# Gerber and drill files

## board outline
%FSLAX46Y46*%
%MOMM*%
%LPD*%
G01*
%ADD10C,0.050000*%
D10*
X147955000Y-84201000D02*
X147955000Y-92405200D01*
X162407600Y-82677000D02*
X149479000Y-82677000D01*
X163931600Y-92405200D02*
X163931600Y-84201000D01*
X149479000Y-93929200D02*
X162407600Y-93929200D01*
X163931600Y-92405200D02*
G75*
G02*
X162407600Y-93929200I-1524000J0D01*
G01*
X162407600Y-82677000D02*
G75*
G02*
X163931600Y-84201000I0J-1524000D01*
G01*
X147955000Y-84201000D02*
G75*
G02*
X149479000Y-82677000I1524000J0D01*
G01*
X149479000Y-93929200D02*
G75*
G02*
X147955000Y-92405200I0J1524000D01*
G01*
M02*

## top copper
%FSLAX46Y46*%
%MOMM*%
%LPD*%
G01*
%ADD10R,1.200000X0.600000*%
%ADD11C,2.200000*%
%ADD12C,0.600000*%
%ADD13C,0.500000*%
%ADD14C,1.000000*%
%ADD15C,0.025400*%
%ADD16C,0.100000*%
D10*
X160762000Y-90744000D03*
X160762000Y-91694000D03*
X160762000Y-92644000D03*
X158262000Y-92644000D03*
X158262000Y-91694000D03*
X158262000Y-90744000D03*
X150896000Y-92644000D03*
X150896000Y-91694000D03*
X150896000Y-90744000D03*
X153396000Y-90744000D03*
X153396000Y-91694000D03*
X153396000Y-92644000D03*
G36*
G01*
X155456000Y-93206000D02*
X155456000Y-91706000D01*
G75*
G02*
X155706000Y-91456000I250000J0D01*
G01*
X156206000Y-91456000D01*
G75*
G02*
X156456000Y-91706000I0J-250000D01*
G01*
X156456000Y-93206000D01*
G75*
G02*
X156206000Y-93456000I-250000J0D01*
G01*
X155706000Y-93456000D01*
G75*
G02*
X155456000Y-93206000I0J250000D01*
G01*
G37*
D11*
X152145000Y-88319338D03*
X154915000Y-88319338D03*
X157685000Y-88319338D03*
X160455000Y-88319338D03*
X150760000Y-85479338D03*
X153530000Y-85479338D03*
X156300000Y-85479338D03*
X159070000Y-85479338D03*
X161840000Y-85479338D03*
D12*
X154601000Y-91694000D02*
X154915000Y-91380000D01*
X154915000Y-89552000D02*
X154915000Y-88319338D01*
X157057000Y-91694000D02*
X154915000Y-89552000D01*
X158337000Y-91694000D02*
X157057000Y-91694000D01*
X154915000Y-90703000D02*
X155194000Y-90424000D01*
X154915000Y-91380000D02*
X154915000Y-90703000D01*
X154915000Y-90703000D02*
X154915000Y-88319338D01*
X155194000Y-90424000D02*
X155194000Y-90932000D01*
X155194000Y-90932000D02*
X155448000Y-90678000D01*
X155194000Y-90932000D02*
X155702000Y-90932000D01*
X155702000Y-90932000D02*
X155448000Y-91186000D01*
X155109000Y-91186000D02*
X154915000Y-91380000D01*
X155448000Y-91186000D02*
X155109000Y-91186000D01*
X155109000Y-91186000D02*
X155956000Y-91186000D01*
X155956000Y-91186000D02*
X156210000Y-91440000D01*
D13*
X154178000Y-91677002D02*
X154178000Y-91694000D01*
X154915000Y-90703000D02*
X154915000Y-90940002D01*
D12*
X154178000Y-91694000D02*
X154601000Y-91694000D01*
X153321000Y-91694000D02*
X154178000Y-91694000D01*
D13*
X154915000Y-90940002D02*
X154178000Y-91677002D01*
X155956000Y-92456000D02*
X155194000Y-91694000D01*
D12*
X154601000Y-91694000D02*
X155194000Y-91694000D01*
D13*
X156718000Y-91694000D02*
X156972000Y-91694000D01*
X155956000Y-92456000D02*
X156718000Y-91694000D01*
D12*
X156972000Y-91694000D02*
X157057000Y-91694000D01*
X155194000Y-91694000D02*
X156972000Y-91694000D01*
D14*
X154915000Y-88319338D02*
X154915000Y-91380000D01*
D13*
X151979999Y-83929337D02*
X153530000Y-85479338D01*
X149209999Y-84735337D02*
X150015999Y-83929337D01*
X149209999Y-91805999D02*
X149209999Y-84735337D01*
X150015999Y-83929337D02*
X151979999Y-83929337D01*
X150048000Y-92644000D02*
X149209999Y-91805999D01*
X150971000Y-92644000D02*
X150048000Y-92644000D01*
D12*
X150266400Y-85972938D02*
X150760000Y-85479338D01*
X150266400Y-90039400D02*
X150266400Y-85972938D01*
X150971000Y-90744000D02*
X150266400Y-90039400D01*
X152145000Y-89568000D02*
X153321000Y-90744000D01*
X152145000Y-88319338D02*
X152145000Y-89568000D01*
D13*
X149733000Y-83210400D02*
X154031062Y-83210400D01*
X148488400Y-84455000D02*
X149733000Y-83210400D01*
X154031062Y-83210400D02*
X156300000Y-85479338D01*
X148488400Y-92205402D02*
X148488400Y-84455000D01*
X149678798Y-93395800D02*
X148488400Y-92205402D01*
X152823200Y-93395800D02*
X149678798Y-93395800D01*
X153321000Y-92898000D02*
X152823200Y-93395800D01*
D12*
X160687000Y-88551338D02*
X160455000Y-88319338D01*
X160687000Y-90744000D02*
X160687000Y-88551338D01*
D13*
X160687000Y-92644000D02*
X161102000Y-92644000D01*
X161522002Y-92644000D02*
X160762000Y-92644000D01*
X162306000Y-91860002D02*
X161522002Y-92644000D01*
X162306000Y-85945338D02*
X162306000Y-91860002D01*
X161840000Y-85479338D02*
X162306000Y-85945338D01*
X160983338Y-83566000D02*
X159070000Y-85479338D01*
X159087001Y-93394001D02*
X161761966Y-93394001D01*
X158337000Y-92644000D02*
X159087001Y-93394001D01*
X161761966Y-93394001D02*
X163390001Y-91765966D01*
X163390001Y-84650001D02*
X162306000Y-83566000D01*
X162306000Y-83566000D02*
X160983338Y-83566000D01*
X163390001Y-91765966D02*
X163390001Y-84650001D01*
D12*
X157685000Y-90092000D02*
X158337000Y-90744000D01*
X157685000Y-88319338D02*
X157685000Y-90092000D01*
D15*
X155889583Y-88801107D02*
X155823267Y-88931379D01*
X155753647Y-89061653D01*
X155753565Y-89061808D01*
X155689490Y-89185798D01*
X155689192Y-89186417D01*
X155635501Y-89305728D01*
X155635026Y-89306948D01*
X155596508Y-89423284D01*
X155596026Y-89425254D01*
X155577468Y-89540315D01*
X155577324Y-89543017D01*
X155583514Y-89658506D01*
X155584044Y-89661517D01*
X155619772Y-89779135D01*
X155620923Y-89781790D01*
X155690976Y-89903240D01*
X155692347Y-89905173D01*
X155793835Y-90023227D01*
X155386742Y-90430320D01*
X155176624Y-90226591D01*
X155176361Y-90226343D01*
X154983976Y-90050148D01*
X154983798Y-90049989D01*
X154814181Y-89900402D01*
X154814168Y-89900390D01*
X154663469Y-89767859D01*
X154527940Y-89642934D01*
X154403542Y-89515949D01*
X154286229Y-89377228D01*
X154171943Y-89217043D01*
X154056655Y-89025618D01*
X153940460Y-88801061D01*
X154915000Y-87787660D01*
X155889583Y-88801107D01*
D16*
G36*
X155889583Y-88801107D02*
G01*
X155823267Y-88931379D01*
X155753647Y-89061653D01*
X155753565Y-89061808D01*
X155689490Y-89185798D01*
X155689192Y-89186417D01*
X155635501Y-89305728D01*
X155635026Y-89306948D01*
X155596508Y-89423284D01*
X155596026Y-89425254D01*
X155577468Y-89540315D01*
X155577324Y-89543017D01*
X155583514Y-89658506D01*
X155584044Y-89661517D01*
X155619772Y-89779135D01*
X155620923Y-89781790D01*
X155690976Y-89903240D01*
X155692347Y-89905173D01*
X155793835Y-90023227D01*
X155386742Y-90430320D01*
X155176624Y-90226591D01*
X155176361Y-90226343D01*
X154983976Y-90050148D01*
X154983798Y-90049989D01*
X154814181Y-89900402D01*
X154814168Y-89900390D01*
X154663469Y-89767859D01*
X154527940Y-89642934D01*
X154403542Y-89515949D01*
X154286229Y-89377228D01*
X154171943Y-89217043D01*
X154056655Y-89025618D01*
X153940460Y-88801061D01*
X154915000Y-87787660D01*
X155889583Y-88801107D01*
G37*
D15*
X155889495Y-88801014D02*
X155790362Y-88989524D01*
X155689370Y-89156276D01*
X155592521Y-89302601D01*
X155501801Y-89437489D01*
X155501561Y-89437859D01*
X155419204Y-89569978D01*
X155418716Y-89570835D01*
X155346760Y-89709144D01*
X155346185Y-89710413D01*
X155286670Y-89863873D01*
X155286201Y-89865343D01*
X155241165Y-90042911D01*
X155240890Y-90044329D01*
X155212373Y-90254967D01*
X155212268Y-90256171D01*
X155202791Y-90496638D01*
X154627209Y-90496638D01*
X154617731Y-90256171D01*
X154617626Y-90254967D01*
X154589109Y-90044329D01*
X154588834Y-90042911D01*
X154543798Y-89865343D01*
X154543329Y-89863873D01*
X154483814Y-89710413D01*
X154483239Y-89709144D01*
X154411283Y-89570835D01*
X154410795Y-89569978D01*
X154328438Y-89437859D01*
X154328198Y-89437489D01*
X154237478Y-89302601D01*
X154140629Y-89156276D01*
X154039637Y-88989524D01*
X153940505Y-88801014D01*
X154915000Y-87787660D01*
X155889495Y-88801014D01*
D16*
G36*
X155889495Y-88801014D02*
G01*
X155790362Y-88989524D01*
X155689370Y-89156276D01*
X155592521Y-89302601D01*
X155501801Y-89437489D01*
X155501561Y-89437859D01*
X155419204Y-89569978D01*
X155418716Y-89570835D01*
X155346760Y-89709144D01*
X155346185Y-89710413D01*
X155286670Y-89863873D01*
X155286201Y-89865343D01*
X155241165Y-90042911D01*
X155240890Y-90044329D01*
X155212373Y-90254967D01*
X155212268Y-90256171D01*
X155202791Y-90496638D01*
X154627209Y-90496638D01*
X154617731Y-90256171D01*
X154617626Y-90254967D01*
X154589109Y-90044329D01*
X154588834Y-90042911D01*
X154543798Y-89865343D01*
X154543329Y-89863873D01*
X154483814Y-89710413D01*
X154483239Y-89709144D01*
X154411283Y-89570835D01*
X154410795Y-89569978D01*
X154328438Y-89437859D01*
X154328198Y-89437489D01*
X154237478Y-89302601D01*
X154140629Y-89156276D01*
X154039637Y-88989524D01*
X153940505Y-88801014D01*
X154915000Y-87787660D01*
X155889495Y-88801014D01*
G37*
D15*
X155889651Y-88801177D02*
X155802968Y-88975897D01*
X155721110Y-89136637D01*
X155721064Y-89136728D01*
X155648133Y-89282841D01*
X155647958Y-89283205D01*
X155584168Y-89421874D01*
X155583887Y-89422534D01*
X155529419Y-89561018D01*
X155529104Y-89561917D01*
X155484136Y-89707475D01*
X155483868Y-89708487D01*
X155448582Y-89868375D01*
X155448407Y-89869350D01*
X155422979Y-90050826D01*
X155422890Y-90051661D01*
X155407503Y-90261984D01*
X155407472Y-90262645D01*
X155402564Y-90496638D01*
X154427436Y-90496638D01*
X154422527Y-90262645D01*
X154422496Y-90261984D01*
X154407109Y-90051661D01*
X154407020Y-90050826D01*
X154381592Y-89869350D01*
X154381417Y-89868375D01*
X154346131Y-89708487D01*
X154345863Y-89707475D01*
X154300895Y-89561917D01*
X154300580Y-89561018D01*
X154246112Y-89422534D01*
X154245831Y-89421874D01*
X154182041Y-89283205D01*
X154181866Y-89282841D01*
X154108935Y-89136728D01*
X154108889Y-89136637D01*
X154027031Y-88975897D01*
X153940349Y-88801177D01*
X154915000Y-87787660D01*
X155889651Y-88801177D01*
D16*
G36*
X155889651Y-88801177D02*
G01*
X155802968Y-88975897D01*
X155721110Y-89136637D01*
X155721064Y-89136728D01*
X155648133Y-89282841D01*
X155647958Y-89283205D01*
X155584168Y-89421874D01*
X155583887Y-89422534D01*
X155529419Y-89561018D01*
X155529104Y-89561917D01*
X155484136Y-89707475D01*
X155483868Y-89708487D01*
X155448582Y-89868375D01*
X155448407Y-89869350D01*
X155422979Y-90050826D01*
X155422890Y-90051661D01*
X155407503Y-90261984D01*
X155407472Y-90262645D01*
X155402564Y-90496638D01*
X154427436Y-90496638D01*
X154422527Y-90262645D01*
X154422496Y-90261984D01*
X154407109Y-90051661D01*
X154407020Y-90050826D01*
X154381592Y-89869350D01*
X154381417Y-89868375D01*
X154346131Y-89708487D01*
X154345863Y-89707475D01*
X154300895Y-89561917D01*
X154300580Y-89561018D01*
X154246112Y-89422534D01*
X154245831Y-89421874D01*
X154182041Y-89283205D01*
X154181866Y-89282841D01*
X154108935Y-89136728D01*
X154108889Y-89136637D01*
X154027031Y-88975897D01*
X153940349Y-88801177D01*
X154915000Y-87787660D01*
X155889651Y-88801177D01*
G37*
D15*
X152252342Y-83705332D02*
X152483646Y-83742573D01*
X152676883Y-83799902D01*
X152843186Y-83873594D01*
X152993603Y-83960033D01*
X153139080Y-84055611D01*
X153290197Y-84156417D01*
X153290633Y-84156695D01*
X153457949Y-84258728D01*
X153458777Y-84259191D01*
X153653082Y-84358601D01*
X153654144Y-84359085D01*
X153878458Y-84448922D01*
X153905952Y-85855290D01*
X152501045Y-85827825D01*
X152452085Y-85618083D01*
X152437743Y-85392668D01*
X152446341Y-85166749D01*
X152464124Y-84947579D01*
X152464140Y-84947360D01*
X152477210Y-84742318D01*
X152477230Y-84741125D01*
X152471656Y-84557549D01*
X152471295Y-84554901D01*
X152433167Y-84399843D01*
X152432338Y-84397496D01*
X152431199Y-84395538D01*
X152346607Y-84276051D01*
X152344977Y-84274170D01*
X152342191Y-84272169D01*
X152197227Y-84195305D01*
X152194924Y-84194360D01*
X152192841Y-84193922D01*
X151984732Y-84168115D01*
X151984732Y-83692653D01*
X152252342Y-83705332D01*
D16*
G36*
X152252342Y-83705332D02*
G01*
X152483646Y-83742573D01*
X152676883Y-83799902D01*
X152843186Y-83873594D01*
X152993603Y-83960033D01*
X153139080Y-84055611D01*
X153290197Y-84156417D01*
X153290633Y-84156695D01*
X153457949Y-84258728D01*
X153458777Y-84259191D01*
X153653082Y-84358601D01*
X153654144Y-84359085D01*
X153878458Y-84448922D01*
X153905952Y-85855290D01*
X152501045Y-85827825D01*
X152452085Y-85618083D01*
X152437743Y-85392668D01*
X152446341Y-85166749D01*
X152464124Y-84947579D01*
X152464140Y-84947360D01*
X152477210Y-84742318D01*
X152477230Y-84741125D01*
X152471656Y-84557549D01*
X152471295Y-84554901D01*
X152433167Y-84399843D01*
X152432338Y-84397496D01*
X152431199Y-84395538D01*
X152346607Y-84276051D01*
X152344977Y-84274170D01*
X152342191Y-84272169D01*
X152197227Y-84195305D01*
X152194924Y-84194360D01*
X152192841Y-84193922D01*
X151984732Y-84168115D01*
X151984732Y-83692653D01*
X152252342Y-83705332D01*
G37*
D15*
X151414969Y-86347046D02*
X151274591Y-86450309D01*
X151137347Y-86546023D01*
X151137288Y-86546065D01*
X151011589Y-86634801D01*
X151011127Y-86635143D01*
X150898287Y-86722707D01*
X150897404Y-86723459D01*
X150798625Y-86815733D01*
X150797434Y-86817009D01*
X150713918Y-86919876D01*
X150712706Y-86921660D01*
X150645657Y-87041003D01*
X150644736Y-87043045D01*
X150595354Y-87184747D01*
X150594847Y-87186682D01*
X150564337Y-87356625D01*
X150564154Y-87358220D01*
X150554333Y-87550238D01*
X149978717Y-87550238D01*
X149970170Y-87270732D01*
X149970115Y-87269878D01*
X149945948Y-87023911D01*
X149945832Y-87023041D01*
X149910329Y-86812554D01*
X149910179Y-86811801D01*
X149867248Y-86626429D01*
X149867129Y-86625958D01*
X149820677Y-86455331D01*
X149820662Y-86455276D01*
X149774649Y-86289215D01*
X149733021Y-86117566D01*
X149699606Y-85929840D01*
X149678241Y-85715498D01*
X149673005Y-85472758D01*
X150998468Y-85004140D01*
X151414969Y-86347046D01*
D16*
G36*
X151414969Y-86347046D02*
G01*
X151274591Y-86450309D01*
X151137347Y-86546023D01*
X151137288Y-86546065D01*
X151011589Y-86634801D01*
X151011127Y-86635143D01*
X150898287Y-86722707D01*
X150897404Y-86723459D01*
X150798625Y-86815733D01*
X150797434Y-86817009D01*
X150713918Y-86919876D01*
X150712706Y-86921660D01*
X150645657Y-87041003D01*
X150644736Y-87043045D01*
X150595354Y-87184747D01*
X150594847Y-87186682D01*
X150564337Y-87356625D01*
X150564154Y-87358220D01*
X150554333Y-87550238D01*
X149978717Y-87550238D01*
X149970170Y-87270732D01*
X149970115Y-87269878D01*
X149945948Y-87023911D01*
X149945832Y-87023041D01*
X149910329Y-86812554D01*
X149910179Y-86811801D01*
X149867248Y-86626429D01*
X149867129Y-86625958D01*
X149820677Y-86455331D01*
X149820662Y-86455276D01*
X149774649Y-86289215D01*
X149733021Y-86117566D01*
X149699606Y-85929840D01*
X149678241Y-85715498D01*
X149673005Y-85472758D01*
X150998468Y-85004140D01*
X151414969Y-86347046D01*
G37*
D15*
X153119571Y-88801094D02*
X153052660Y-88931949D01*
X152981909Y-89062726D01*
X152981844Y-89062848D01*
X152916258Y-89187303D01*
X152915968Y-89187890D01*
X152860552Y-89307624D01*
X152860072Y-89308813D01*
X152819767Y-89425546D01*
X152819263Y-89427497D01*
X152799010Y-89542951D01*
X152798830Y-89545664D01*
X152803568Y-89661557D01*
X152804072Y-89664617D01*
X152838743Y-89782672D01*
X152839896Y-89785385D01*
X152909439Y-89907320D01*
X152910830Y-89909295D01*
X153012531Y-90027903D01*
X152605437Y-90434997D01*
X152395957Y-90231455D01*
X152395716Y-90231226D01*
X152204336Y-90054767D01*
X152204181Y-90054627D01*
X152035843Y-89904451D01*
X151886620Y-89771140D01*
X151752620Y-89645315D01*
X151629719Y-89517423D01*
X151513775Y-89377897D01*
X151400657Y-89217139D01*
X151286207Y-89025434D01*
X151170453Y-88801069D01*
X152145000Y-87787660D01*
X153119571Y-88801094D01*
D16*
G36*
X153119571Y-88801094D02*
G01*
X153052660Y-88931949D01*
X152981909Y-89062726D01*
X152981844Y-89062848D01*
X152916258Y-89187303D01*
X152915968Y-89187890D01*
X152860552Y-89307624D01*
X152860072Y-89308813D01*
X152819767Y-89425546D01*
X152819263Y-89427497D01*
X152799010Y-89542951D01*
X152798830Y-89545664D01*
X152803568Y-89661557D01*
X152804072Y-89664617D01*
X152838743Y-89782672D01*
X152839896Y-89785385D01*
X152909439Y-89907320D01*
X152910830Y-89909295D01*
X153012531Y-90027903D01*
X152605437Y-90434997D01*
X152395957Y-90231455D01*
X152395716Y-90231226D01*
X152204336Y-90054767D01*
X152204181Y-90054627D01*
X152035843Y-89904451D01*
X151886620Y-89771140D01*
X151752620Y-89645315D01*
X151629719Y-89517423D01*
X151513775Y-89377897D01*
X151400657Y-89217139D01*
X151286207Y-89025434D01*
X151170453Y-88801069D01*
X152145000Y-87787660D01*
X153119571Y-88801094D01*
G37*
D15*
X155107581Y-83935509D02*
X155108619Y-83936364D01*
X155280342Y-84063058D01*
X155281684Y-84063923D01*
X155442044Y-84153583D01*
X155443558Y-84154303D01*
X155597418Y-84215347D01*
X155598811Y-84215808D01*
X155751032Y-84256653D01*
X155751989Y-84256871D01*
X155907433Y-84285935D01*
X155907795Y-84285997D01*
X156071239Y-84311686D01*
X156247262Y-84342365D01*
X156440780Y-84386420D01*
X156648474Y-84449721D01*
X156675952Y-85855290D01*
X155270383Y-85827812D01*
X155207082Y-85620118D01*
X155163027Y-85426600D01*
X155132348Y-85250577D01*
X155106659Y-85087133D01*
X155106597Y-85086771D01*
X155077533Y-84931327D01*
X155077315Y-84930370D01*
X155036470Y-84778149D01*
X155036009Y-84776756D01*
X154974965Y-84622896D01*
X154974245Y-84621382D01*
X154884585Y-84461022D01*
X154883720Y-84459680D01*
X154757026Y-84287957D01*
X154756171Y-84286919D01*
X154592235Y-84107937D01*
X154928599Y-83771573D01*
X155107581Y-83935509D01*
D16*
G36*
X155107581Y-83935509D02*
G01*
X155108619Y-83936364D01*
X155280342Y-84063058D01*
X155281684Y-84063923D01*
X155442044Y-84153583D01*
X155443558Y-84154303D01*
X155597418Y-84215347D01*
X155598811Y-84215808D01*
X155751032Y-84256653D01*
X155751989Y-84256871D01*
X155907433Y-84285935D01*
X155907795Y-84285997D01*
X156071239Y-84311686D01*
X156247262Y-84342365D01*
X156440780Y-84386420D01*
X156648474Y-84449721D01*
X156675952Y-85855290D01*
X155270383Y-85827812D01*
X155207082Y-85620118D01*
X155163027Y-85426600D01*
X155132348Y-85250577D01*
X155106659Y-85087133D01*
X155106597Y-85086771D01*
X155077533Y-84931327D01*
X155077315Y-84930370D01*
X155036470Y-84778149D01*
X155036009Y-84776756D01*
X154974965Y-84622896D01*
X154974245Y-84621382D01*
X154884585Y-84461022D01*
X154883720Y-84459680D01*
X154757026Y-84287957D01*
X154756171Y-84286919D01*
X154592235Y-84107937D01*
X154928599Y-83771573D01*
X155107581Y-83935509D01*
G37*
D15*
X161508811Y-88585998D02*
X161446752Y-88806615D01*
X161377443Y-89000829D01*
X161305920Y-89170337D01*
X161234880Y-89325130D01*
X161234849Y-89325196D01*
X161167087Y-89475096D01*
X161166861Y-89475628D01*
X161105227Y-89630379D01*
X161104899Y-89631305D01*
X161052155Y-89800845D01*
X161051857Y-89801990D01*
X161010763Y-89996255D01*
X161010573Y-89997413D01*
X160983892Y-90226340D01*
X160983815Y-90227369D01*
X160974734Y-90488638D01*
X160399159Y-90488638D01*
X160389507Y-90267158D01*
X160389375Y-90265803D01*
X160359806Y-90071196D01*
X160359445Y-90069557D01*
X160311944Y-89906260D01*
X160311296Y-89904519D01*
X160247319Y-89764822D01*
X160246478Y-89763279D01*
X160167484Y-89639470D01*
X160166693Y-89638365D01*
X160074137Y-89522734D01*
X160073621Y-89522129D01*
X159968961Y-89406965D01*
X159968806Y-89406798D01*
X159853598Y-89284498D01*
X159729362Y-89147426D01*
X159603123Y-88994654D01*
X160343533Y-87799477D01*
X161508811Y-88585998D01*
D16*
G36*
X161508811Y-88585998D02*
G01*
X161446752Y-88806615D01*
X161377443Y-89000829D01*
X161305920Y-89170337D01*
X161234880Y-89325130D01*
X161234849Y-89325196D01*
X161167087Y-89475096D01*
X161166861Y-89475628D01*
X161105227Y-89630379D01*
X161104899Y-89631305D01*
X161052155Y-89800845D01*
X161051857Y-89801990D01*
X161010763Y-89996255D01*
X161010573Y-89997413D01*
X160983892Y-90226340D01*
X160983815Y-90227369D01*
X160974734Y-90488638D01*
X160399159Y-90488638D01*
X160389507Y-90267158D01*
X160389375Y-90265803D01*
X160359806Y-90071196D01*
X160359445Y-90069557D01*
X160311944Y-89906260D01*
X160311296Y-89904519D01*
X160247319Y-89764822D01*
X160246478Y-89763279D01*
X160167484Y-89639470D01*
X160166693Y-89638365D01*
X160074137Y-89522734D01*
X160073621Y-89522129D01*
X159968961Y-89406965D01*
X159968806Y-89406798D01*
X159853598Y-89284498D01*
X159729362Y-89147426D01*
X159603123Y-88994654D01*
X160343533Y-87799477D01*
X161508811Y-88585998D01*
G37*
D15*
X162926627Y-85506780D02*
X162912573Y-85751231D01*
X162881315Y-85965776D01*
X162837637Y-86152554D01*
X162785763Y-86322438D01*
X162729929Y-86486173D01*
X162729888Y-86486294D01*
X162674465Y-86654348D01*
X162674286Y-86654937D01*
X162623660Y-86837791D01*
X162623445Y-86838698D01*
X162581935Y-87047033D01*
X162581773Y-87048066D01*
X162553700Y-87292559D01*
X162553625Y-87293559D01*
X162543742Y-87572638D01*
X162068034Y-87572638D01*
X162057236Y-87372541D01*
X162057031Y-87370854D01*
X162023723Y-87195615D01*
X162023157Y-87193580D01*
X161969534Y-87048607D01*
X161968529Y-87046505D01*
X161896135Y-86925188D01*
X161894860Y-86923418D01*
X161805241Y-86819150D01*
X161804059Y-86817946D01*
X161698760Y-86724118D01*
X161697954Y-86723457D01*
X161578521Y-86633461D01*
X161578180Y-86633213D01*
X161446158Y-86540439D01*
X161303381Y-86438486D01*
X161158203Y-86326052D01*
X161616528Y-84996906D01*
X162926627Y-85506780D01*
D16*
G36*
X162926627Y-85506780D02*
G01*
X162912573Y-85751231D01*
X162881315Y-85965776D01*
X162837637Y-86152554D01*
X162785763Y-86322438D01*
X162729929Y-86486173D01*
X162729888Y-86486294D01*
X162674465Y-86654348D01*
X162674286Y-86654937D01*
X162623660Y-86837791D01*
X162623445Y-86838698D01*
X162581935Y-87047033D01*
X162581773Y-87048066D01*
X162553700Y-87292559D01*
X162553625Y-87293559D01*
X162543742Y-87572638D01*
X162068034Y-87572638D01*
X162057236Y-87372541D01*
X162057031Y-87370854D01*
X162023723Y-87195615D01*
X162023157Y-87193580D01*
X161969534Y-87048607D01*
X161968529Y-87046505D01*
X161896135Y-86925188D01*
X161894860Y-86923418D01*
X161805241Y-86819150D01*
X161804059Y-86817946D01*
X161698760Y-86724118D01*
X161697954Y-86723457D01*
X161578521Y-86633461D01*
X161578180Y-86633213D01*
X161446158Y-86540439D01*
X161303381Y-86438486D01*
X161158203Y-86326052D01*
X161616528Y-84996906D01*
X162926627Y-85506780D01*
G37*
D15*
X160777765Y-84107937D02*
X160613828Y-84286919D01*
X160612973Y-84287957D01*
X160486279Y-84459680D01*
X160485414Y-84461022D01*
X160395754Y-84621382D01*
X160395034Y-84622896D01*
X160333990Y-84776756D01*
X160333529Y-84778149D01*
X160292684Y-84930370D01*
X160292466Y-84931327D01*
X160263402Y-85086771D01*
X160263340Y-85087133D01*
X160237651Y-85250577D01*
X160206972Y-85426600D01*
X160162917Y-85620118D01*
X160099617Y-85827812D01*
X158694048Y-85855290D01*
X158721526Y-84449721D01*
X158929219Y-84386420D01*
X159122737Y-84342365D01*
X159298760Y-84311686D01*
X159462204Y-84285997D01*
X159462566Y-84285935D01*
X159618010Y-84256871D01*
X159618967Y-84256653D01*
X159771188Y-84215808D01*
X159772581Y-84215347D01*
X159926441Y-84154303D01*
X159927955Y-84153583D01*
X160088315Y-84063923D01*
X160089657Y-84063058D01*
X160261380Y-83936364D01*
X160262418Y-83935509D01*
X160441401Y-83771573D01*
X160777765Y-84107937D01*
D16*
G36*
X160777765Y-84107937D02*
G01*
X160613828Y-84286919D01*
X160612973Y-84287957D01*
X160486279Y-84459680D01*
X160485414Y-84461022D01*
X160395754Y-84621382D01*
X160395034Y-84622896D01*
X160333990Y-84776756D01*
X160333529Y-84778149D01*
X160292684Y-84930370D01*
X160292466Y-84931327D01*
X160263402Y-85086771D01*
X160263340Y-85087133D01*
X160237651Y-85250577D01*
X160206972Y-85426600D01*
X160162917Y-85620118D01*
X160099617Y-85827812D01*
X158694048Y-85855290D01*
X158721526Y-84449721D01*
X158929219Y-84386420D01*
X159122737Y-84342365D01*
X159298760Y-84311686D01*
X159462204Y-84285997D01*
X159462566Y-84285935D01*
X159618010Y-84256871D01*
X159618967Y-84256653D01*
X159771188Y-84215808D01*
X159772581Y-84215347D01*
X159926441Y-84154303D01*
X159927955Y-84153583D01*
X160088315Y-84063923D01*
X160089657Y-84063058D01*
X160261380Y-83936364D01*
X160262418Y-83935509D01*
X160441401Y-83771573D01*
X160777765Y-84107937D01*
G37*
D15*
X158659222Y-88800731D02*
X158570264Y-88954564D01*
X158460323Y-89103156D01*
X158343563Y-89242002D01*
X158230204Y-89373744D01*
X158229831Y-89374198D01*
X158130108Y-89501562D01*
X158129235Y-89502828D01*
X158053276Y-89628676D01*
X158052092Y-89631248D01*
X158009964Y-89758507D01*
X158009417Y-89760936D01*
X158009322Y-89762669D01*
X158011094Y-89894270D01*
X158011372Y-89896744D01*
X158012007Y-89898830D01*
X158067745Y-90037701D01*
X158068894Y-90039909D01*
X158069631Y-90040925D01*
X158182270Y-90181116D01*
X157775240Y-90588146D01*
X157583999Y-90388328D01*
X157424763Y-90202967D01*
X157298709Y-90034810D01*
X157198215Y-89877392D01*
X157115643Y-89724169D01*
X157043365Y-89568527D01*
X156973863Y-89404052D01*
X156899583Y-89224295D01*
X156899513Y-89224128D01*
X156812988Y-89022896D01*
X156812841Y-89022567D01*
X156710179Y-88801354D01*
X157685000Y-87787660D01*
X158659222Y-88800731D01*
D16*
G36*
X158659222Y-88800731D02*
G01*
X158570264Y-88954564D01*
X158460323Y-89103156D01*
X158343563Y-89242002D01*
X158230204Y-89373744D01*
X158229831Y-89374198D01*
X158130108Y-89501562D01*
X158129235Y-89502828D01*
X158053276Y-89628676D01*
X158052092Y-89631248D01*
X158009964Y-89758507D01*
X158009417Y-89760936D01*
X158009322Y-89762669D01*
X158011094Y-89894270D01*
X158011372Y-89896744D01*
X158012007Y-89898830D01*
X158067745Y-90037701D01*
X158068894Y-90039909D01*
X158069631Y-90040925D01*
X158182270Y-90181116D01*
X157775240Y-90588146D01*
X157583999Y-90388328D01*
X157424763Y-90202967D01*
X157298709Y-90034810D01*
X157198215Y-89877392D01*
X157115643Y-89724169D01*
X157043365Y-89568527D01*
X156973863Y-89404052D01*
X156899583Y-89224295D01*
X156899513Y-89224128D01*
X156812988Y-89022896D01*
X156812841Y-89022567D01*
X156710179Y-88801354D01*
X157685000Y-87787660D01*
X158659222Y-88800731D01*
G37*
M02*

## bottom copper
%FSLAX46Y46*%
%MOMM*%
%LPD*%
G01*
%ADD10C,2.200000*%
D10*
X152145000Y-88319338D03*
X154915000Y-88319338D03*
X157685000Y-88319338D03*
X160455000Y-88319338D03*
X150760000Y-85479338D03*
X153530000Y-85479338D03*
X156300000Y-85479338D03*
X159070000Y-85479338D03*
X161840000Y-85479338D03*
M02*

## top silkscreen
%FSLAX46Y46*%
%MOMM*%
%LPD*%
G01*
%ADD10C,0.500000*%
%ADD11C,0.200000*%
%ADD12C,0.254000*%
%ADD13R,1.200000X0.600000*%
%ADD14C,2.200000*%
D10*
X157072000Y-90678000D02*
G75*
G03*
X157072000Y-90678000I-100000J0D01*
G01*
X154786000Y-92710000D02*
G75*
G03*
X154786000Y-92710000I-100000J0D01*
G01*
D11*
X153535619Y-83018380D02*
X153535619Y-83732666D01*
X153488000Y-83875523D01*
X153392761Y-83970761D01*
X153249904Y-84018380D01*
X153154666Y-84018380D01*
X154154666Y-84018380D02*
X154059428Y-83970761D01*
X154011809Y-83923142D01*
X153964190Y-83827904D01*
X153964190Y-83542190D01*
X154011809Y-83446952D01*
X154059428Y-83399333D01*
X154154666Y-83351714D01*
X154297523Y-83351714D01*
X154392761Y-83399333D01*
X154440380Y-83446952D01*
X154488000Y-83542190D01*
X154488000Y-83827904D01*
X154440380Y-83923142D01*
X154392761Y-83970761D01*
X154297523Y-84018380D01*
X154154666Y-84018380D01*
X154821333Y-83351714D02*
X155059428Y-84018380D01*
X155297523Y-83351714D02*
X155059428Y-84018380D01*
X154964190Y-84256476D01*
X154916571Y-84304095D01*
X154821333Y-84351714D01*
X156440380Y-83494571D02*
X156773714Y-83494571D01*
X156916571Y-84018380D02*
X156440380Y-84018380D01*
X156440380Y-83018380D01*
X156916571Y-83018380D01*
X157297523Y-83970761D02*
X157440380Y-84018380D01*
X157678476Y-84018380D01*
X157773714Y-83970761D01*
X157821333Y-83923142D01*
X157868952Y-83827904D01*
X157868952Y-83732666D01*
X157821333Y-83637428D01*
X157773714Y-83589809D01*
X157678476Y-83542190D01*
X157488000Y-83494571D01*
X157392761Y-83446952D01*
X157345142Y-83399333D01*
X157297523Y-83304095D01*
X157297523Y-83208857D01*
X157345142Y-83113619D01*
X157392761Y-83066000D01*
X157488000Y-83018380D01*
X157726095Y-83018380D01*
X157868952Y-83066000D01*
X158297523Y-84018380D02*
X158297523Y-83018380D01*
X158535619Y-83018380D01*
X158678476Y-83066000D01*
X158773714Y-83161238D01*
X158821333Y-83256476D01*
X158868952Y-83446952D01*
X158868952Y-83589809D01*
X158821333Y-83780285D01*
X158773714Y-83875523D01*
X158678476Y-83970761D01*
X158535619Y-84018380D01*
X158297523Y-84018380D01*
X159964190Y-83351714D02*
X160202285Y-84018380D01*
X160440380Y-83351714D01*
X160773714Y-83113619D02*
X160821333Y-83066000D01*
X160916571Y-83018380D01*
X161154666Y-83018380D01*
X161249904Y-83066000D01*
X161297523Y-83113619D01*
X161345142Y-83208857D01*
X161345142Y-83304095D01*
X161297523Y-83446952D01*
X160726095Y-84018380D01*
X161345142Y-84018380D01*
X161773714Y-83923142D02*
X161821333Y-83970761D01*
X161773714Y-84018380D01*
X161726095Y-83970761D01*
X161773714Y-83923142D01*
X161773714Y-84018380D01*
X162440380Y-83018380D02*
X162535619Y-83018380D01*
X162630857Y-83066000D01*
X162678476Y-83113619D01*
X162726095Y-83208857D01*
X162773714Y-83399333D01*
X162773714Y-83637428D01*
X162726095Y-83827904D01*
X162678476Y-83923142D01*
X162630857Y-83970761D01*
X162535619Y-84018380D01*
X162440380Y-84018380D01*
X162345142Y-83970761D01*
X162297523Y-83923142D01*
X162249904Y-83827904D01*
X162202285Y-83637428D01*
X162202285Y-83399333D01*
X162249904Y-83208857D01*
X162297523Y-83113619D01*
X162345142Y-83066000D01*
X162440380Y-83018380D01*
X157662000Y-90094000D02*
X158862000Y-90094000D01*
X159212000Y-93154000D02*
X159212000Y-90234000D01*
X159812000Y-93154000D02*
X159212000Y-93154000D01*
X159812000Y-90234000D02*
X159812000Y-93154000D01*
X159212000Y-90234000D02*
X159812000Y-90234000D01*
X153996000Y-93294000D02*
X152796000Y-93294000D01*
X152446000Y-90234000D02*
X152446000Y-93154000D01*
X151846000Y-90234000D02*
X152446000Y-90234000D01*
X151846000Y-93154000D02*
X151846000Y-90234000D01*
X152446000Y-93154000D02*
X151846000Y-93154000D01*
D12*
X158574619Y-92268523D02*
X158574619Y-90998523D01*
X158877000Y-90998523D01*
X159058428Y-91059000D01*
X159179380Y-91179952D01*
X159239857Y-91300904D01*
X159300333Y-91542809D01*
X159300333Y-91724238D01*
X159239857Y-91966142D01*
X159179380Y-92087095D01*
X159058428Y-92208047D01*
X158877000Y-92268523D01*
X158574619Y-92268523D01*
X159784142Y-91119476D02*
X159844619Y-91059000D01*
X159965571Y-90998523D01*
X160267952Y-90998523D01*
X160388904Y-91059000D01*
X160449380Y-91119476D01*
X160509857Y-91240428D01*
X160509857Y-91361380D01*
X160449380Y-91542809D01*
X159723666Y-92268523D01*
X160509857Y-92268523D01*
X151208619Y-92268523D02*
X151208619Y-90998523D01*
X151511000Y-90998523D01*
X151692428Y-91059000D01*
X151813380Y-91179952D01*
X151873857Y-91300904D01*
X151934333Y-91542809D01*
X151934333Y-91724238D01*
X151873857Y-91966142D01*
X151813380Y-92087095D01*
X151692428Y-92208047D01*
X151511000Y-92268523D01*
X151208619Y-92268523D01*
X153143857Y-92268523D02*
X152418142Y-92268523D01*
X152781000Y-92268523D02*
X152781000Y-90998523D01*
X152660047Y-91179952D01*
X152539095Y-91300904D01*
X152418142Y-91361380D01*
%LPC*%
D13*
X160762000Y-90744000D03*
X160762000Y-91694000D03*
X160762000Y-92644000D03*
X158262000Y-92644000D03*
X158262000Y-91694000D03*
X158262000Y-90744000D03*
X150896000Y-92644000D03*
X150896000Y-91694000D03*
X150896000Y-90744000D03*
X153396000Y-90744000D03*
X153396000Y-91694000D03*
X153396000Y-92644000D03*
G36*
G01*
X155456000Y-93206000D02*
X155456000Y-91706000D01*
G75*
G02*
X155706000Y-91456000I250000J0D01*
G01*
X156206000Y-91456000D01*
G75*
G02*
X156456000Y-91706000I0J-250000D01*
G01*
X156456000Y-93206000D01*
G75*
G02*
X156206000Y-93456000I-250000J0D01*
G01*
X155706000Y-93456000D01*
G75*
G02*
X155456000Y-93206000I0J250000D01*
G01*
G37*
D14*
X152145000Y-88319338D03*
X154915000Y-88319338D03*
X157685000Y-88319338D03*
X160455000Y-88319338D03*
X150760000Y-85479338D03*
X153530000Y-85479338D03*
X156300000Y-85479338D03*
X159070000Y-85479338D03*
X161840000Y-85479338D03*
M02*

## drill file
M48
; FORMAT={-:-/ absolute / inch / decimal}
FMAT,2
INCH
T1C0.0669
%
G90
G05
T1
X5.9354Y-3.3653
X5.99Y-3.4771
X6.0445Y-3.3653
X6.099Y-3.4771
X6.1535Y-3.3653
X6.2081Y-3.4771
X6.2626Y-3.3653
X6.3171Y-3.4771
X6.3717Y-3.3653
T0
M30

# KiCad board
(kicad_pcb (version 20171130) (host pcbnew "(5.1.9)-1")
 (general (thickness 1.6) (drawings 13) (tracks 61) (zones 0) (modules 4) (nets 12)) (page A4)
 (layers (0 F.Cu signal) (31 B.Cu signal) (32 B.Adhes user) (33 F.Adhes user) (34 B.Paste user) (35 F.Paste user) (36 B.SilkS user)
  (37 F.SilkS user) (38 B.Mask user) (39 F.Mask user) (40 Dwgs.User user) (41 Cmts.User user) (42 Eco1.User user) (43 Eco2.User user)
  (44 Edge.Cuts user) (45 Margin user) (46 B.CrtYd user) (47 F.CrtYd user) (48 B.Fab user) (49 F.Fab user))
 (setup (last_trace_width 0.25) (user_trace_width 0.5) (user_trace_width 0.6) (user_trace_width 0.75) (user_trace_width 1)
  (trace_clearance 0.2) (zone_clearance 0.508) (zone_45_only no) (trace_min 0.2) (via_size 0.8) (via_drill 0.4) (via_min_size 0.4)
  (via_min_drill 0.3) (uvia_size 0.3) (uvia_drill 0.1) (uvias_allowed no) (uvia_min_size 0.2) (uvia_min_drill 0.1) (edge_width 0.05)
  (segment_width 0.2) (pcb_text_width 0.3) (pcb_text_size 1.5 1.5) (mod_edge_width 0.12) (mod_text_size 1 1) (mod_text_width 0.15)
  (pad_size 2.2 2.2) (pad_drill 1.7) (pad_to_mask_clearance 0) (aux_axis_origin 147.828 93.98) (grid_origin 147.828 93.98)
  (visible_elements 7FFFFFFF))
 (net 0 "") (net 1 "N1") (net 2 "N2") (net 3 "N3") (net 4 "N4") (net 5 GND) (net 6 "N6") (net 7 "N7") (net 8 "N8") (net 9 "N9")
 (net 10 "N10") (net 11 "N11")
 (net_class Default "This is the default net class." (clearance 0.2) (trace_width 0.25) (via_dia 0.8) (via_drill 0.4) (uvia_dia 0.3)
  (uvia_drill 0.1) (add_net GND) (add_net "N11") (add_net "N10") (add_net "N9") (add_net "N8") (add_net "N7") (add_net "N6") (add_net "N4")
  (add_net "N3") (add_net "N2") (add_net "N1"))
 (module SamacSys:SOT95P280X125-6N (layer F.Cu) (at 159.512 91.694)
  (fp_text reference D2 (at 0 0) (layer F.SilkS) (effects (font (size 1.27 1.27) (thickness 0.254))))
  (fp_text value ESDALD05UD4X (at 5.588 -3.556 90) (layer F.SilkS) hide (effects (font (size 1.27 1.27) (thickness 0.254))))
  (fp_line (start -1.85 -1.6) (end -0.65 -1.6) (layer F.SilkS) (width 0.2))
  (fp_line (start -0.3 1.46) (end -0.3 -1.46) (layer F.SilkS) (width 0.2))
  (fp_line (start 0.3 1.46) (end -0.3 1.46) (layer F.SilkS) (width 0.2))
  (fp_line (start 0.3 -1.46) (end 0.3 1.46) (layer F.SilkS) (width 0.2))
  (fp_line (start -0.3 -1.46) (end 0.3 -1.46) (layer F.SilkS) (width 0.2))
  (pad 6 smd rect (at 1.25 -0.95 90) (size 0.6 1.2) (layers F.Cu F.Paste F.Mask) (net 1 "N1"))
  (pad 5 smd rect (at 1.25 0 90) (size 0.6 1.2) (layers F.Cu F.Paste F.Mask) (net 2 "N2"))
  (pad 4 smd rect (at 1.25 0.95 90) (size 0.6 1.2) (layers F.Cu F.Paste F.Mask) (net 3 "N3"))
  (pad 3 smd rect (at -1.25 0.95 90) (size 0.6 1.2) (layers F.Cu F.Paste F.Mask) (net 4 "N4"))
  (pad 2 smd rect (at -1.25 0 90) (size 0.6 1.2) (layers F.Cu F.Paste F.Mask) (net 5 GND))
  (pad 1 smd rect (at -1.25 -0.95 90) (size 0.6 1.2) (layers F.Cu F.Paste F.Mask) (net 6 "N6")))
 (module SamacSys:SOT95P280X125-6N (layer F.Cu) (at 152.146 91.694 180)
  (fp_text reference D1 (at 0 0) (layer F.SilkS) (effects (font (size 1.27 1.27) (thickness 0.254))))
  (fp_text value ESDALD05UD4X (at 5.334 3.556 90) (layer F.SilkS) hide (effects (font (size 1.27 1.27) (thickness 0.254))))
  (fp_line (start -1.85 -1.6) (end -0.65 -1.6) (layer F.SilkS) (width 0.2))
  (fp_line (start -0.3 1.46) (end -0.3 -1.46) (layer F.SilkS) (width 0.2))
  (fp_line (start 0.3 1.46) (end -0.3 1.46) (layer F.SilkS) (width 0.2))
  (fp_line (start 0.3 -1.46) (end 0.3 1.46) (layer F.SilkS) (width 0.2))
  (fp_line (start -0.3 -1.46) (end 0.3 -1.46) (layer F.SilkS) (width 0.2))
  (pad 6 smd rect (at 1.25 -0.95 270) (size 0.6 1.2) (layers F.Cu F.Paste F.Mask) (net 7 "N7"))
  (pad 5 smd rect (at 1.25 0 270) (size 0.6 1.2) (layers F.Cu F.Paste F.Mask) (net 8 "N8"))
  (pad 4 smd rect (at 1.25 0.95 270) (size 0.6 1.2) (layers F.Cu F.Paste F.Mask) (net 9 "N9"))
  (pad 3 smd rect (at -1.25 0.95 270) (size 0.6 1.2) (layers F.Cu F.Paste F.Mask) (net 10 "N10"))
  (pad 2 smd rect (at -1.25 0 270) (size 0.6 1.2) (layers F.Cu F.Paste F.Mask) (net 5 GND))
  (pad 1 smd rect (at -1.25 -0.95 270) (size 0.6 1.2) (layers F.Cu F.Paste F.Mask) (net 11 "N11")))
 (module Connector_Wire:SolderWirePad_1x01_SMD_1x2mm (layer F.Cu) (at 155.956 92.456)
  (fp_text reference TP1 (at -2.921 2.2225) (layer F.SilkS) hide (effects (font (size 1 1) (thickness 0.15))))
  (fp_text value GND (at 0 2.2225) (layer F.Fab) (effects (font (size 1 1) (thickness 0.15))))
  (pad 1 smd roundrect (at 0 0) (size 1 2) (layers F.Cu F.Paste F.Mask) (roundrect_rratio 0.25) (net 5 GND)))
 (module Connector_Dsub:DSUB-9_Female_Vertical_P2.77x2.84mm (layer F.Cu) (at 161.84 85.479338)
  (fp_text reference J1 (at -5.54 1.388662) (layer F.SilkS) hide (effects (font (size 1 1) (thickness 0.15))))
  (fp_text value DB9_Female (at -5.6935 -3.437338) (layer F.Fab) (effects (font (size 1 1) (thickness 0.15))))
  (pad 9 thru_hole circle (at -9.695 2.84) (size 2.2 2.2) (drill 1.7) (layers *.Cu *.Mask) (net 10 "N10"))
  (pad 8 thru_hole circle (at -6.925 2.84) (size 2.2 2.2) (drill 1.7) (layers *.Cu *.Mask) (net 5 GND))
  (pad 7 thru_hole circle (at -4.155 2.84) (size 2.2 2.2) (drill 1.7) (layers *.Cu *.Mask) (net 6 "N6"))
  (pad 6 thru_hole circle (at -1.385 2.84) (size 2.2 2.2) (drill 1.7) (layers *.Cu *.Mask) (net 1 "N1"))
  (pad 5 thru_hole circle (at -11.08 0) (size 2.2 2.2) (drill 1.7) (layers *.Cu *.Mask) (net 9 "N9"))
  (pad 4 thru_hole circle (at -8.31 0) (size 2.2 2.2) (drill 1.7) (layers *.Cu *.Mask) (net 7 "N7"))
  (pad 3 thru_hole circle (at -5.54 0) (size 2.2 2.2) (drill 1.7) (layers *.Cu *.Mask) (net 11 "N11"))
  (pad 2 thru_hole circle (at -2.77 0) (size 2.2 2.2) (drill 1.7) (layers *.Cu *.Mask) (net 4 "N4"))
  (pad 1 thru_hole circle (at 0 0) (size 2.2 2.2) (drill 1.7) (layers *.Cu *.Mask) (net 3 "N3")))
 (gr_circle (center 156.972 90.678) (end 157.072 90.678) (layer F.SilkS) (width 0.5))
 (gr_circle (center 154.686 92.71) (end 154.786 92.71) (layer F.SilkS) (width 0.5))
 (gr_line (start 147.955 84.201) (end 147.955 92.4052) (layer Edge.Cuts) (width 0.05))
 (gr_line (start 162.4076 82.677) (end 149.479 82.677) (layer Edge.Cuts) (width 0.05))
 (gr_line (start 163.9316 92.4052) (end 163.9316 84.201) (layer Edge.Cuts) (width 0.05))
 (gr_line (start 149.479 93.9292) (end 162.4076 93.9292) (layer Edge.Cuts) (width 0.05))
 (gr_arc (start 162.4076 92.4052) (end 162.4076 93.9292) (angle -90) (layer Edge.Cuts) (width 0.05))
 (gr_arc (start 162.4076 84.201) (end 163.9316 84.201) (angle -90) (layer Edge.Cuts) (width 0.05))
 (gr_arc (start 149.479 84.201) (end 149.479 82.677) (angle -90) (layer Edge.Cuts) (width 0.05))
 (gr_arc (start 149.479 92.4052) (end 147.955 92.4052) (angle -90) (layer Edge.Cuts) (width 0.05))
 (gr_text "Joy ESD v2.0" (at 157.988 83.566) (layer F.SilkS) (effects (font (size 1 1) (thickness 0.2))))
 (segment (start 154.601 91.694) (end 154.915 91.38) (width 0.6) (layer F.Cu) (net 5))
 (segment (start 154.915 89.552) (end 154.915 88.319338) (width 0.6) (layer F.Cu) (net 5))
 (segment (start 157.057 91.694) (end 154.915 89.552) (width 0.6) (layer F.Cu) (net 5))
 (segment (start 158.337 91.694) (end 157.057 91.694) (width 0.6) (layer F.Cu) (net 5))
 (segment (start 154.915 90.703) (end 155.194 90.424) (width 0.6) (layer F.Cu) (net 5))
 (segment (start 154.915 91.38) (end 154.915 90.703) (width 0.6) (layer F.Cu) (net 5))
 (segment (start 154.915 90.703) (end 154.915 88.319338) (width 0.6) (layer F.Cu) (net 5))
 (segment (start 155.194 90.424) (end 155.194 90.932) (width 0.6) (layer F.Cu) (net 5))
 (segment (start 155.194 90.932) (end 155.448 90.678) (width 0.6) (layer F.Cu) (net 5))
 (segment (start 155.194 90.932) (end 155.702 90.932) (width 0.6) (layer F.Cu) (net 5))
 (segment (start 155.702 90.932) (end 155.448 91.186) (width 0.6) (layer F.Cu) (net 5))
 (segment (start 155.109 91.186) (end 154.915 91.38) (width 0.6) (layer F.Cu) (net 5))
 (segment (start 155.448 91.186) (end 155.109 91.186) (width 0.6) (layer F.Cu) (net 5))
 (segment (start 155.109 91.186) (end 155.956 91.186) (width 0.6) (layer F.Cu) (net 5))
 (segment (start 155.956 91.186) (end 156.21 91.44) (width 0.6) (layer F.Cu) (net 5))
 (segment (start 154.178 91.677002) (end 154.178 91.694) (width 0.5) (layer F.Cu) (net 5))
 (segment (start 154.915 90.703) (end 154.915 90.940002) (width 0.5) (layer F.Cu) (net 5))
 (segment (start 154.178 91.694) (end 154.601 91.694) (width 0.6) (layer F.Cu) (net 5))
 (segment (start 153.321 91.694) (end 154.178 91.694) (width 0.6) (layer F.Cu) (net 5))
 (segment (start 154.915 90.940002) (end 154.178 91.677002) (width 0.5) (layer F.Cu) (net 5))
 (segment (start 155.956 92.456) (end 155.194 91.694) (width 0.5) (layer F.Cu) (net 5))
 (segment (start 154.601 91.694) (end 155.194 91.694) (width 0.6) (layer F.Cu) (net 5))
 (segment (start 156.718 91.694) (end 156.972 91.694) (width 0.5) (layer F.Cu) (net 5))
 (segment (start 155.956 92.456) (end 156.718 91.694) (width 0.5) (layer F.Cu) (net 5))
 (segment (start 156.972 91.694) (end 157.057 91.694) (width 0.6) (layer F.Cu) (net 5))
 (segment (start 155.194 91.694) (end 156.972 91.694) (width 0.6) (layer F.Cu) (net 5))
 (segment (start 154.915 88.319338) (end 154.915 91.38) (width 1) (layer F.Cu) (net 5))
 (segment (start 151.979999 83.929337) (end 153.53 85.479338) (width 0.5) (layer F.Cu) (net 7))
 (segment (start 149.209999 84.735337) (end 150.015999 83.929337) (width 0.5) (layer F.Cu) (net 7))
 (segment (start 149.209999 91.805999) (end 149.209999 84.735337) (width 0.5) (layer F.Cu) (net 7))
 (segment (start 150.015999 83.929337) (end 151.979999 83.929337) (width 0.5) (layer F.Cu) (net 7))
 (segment (start 150.048 92.644) (end 149.209999 91.805999) (width 0.5) (layer F.Cu) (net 7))
 (segment (start 150.971 92.644) (end 150.048 92.644) (width 0.5) (layer F.Cu) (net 7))
 (segment (start 150.2664 85.972938) (end 150.76 85.479338) (width 0.6) (layer F.Cu) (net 9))
 (segment (start 150.2664 90.0394) (end 150.2664 85.972938) (width 0.6) (layer F.Cu) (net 9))
 (segment (start 150.971 90.744) (end 150.2664 90.0394) (width 0.6) (layer F.Cu) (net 9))
 (segment (start 152.145 89.568) (end 153.321 90.744) (width 0.6) (layer F.Cu) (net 10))
 (segment (start 152.145 88.319338) (end 152.145 89.568) (width 0.6) (layer F.Cu) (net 10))
 (segment (start 149.733 83.2104) (end 154.031062 83.2104) (width 0.5) (layer F.Cu) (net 11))
 (segment (start 148.4884 84.455) (end 149.733 83.2104) (width 0.5) (layer F.Cu) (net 11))
 (segment (start 154.031062 83.2104) (end 156.3 85.479338) (width 0.5) (layer F.Cu) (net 11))
 (segment (start 148.4884 92.205402) (end 148.4884 84.455) (width 0.5) (layer F.Cu) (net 11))
 (segment (start 149.678798 93.3958) (end 148.4884 92.205402) (width 0.5) (layer F.Cu) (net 11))
 (segment (start 152.8232 93.3958) (end 149.678798 93.3958) (width 0.5) (layer F.Cu) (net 11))
 (segment (start 153.321 92.898) (end 152.8232 93.3958) (width 0.5) (layer F.Cu) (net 11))
 (segment (start 160.687 88.551338) (end 160.455 88.319338) (width 0.6) (layer F.Cu) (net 1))
 (segment (start 160.687 90.744) (end 160.687 88.551338) (width 0.6) (layer F.Cu) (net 1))
 (segment (start 160.687 92.644) (end 161.102 92.644) (width 0.5) (layer F.Cu) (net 3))
 (segment (start 161.522002 92.644) (end 160.762 92.644) (width 0.5) (layer F.Cu) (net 3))
 (segment (start 162.306 91.860002) (end 161.522002 92.644) (width 0.5) (layer F.Cu) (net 3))
 (segment (start 162.306 85.945338) (end 162.306 91.860002) (width 0.5) (layer F.Cu) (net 3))
 (segment (start 161.84 85.479338) (end 162.306 85.945338) (width 0.5) (layer F.Cu) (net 3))
 (segment (start 160.983338 83.566) (end 159.07 85.479338) (width 0.5) (layer F.Cu) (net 4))
 (segment (start 159.087001 93.394001) (end 161.761966 93.394001) (width 0.5) (layer F.Cu) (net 4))
 (segment (start 158.337 92.644) (end 159.087001 93.394001) (width 0.5) (layer F.Cu) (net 4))
 (segment (start 161.761966 93.394001) (end 163.390001 91.765966) (width 0.5) (layer F.Cu) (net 4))
 (segment (start 163.390001 84.650001) (end 162.306 83.566) (width 0.5) (layer F.Cu) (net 4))
 (segment (start 162.306 83.566) (end 160.983338 83.566) (width 0.5) (layer F.Cu) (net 4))
 (segment (start 163.390001 91.765966) (end 163.390001 84.650001) (width 0.5) (layer F.Cu) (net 4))
 (segment (start 157.685 90.092) (end 158.337 90.744) (width 0.6) (layer F.Cu) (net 6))
 (segment (start 157.685 88.319338) (end 157.685 90.092) (width 0.6) (layer F.Cu) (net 6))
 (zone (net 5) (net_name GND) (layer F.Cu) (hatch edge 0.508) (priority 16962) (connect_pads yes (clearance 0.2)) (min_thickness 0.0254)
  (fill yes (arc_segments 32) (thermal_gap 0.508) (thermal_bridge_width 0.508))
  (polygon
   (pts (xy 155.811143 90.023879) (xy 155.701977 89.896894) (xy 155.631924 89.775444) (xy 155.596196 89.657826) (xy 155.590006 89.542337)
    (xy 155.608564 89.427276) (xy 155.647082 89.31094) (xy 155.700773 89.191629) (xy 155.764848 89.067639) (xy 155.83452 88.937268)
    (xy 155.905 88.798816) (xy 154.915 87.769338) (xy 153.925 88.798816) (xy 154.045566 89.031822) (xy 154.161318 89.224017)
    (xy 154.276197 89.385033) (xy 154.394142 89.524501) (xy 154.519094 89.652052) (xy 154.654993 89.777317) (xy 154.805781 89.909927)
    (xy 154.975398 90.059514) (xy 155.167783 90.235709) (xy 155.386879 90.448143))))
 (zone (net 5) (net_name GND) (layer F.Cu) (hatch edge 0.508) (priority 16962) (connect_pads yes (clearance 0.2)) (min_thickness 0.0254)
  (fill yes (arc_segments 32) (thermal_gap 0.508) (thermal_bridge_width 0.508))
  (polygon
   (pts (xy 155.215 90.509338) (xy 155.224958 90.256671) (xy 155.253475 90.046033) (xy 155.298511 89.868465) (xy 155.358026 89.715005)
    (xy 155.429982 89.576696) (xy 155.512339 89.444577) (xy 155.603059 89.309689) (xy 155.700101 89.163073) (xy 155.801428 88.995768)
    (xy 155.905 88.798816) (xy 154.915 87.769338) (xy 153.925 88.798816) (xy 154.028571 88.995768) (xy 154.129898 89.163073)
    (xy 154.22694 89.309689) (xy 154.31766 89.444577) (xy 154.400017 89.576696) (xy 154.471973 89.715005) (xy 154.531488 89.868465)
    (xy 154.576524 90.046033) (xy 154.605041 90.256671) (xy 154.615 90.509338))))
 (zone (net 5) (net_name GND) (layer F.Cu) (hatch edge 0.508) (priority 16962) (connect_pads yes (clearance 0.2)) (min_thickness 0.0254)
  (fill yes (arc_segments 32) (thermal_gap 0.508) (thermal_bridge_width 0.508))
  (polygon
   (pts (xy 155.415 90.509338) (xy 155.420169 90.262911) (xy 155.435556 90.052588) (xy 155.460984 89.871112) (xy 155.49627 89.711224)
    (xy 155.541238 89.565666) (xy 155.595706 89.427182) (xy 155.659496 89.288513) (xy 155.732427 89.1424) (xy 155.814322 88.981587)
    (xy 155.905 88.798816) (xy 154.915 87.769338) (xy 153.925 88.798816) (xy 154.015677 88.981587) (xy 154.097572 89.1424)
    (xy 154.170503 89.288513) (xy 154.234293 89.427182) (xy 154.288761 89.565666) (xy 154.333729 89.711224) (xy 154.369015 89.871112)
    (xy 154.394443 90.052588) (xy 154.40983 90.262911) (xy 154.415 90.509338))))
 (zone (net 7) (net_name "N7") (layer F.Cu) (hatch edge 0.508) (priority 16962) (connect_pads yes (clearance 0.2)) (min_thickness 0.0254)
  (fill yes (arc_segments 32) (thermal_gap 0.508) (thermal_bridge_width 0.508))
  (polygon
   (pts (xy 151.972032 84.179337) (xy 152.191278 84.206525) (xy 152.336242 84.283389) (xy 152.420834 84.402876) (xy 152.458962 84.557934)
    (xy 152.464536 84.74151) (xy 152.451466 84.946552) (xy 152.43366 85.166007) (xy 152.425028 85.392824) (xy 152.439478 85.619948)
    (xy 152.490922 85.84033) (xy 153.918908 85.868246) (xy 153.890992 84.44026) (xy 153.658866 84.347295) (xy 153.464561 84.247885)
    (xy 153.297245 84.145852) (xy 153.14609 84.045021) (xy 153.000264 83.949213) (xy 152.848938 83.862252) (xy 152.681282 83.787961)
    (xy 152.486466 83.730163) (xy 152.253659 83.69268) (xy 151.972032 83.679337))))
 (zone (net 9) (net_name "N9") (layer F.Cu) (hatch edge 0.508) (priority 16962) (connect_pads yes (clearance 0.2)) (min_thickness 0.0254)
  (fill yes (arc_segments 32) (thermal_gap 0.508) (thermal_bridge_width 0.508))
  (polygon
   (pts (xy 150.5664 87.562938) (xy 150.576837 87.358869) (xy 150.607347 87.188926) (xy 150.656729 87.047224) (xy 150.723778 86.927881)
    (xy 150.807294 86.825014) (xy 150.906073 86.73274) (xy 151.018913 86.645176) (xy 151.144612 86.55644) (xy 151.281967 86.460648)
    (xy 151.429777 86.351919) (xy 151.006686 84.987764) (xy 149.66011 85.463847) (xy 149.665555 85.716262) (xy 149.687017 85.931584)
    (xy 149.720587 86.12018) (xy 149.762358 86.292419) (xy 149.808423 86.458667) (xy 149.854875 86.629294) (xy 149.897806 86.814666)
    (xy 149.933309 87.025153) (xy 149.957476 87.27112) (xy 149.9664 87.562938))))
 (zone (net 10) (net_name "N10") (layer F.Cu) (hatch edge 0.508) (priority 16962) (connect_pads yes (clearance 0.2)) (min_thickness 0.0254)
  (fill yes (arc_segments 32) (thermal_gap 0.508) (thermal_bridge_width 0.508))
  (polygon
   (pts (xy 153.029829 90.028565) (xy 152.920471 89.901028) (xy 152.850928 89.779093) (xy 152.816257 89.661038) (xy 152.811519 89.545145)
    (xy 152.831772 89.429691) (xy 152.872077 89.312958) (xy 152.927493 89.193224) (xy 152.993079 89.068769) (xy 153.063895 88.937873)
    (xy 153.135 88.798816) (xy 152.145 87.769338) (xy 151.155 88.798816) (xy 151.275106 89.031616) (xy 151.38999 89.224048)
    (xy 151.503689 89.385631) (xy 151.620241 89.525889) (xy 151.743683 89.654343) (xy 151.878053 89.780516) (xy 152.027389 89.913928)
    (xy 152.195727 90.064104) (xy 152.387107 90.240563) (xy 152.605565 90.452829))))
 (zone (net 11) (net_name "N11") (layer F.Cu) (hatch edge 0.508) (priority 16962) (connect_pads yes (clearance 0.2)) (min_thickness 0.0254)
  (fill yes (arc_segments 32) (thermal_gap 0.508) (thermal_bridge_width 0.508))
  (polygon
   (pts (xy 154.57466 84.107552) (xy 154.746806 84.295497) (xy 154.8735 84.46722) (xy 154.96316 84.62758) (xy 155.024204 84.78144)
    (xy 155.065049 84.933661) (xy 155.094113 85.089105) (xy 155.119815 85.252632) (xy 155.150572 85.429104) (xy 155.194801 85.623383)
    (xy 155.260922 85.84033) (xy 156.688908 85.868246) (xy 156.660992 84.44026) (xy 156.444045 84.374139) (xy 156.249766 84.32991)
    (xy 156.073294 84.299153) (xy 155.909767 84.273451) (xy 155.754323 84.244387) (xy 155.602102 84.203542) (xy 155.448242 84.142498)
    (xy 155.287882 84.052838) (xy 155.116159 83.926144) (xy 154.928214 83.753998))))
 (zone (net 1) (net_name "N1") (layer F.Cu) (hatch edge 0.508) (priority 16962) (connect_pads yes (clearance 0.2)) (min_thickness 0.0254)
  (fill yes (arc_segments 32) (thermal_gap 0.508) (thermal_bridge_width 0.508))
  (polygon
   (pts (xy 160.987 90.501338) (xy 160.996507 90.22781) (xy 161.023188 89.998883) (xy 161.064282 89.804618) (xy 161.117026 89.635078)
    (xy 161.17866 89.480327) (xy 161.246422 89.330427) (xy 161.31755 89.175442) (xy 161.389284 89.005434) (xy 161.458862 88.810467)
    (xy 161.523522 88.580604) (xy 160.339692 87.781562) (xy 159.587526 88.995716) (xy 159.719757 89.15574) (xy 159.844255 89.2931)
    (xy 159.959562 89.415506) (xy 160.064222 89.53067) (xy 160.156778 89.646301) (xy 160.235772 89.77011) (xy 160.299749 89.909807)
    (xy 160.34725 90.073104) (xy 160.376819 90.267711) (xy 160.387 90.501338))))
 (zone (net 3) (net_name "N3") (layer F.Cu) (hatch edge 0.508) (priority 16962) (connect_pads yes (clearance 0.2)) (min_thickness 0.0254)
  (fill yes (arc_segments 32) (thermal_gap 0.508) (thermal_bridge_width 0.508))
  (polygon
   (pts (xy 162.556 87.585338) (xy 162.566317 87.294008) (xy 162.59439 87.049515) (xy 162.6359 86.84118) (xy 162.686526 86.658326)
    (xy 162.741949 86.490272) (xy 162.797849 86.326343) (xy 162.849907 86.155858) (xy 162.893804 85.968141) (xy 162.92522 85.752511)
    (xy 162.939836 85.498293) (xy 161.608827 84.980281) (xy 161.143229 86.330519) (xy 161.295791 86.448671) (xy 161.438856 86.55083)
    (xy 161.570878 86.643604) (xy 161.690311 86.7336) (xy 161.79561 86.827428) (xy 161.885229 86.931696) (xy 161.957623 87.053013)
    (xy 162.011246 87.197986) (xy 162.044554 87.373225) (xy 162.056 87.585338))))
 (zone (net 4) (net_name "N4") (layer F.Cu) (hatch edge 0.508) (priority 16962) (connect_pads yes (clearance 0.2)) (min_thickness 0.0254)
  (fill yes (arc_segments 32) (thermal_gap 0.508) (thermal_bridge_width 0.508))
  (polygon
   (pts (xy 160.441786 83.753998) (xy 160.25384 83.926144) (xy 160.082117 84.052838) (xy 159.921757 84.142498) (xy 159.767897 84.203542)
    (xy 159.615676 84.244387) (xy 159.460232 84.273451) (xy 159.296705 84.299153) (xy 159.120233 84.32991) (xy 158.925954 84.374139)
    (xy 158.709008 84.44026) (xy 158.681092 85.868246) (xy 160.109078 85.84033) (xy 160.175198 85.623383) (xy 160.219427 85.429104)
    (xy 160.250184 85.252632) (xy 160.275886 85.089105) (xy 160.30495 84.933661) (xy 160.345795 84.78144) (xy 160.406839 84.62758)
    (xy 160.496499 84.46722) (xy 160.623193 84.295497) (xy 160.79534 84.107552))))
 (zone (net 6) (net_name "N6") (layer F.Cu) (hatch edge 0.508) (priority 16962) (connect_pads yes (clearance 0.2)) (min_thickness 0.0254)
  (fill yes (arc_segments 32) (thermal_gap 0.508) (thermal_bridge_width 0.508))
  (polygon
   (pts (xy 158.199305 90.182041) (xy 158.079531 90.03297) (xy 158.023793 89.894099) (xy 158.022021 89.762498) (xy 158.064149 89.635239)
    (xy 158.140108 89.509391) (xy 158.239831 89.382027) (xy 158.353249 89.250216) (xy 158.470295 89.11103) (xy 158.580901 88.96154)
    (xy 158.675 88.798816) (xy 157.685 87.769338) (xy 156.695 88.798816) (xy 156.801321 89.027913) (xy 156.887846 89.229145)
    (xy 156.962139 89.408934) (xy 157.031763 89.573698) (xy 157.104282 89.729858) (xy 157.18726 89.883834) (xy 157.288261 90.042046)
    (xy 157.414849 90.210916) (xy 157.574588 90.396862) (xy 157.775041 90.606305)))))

